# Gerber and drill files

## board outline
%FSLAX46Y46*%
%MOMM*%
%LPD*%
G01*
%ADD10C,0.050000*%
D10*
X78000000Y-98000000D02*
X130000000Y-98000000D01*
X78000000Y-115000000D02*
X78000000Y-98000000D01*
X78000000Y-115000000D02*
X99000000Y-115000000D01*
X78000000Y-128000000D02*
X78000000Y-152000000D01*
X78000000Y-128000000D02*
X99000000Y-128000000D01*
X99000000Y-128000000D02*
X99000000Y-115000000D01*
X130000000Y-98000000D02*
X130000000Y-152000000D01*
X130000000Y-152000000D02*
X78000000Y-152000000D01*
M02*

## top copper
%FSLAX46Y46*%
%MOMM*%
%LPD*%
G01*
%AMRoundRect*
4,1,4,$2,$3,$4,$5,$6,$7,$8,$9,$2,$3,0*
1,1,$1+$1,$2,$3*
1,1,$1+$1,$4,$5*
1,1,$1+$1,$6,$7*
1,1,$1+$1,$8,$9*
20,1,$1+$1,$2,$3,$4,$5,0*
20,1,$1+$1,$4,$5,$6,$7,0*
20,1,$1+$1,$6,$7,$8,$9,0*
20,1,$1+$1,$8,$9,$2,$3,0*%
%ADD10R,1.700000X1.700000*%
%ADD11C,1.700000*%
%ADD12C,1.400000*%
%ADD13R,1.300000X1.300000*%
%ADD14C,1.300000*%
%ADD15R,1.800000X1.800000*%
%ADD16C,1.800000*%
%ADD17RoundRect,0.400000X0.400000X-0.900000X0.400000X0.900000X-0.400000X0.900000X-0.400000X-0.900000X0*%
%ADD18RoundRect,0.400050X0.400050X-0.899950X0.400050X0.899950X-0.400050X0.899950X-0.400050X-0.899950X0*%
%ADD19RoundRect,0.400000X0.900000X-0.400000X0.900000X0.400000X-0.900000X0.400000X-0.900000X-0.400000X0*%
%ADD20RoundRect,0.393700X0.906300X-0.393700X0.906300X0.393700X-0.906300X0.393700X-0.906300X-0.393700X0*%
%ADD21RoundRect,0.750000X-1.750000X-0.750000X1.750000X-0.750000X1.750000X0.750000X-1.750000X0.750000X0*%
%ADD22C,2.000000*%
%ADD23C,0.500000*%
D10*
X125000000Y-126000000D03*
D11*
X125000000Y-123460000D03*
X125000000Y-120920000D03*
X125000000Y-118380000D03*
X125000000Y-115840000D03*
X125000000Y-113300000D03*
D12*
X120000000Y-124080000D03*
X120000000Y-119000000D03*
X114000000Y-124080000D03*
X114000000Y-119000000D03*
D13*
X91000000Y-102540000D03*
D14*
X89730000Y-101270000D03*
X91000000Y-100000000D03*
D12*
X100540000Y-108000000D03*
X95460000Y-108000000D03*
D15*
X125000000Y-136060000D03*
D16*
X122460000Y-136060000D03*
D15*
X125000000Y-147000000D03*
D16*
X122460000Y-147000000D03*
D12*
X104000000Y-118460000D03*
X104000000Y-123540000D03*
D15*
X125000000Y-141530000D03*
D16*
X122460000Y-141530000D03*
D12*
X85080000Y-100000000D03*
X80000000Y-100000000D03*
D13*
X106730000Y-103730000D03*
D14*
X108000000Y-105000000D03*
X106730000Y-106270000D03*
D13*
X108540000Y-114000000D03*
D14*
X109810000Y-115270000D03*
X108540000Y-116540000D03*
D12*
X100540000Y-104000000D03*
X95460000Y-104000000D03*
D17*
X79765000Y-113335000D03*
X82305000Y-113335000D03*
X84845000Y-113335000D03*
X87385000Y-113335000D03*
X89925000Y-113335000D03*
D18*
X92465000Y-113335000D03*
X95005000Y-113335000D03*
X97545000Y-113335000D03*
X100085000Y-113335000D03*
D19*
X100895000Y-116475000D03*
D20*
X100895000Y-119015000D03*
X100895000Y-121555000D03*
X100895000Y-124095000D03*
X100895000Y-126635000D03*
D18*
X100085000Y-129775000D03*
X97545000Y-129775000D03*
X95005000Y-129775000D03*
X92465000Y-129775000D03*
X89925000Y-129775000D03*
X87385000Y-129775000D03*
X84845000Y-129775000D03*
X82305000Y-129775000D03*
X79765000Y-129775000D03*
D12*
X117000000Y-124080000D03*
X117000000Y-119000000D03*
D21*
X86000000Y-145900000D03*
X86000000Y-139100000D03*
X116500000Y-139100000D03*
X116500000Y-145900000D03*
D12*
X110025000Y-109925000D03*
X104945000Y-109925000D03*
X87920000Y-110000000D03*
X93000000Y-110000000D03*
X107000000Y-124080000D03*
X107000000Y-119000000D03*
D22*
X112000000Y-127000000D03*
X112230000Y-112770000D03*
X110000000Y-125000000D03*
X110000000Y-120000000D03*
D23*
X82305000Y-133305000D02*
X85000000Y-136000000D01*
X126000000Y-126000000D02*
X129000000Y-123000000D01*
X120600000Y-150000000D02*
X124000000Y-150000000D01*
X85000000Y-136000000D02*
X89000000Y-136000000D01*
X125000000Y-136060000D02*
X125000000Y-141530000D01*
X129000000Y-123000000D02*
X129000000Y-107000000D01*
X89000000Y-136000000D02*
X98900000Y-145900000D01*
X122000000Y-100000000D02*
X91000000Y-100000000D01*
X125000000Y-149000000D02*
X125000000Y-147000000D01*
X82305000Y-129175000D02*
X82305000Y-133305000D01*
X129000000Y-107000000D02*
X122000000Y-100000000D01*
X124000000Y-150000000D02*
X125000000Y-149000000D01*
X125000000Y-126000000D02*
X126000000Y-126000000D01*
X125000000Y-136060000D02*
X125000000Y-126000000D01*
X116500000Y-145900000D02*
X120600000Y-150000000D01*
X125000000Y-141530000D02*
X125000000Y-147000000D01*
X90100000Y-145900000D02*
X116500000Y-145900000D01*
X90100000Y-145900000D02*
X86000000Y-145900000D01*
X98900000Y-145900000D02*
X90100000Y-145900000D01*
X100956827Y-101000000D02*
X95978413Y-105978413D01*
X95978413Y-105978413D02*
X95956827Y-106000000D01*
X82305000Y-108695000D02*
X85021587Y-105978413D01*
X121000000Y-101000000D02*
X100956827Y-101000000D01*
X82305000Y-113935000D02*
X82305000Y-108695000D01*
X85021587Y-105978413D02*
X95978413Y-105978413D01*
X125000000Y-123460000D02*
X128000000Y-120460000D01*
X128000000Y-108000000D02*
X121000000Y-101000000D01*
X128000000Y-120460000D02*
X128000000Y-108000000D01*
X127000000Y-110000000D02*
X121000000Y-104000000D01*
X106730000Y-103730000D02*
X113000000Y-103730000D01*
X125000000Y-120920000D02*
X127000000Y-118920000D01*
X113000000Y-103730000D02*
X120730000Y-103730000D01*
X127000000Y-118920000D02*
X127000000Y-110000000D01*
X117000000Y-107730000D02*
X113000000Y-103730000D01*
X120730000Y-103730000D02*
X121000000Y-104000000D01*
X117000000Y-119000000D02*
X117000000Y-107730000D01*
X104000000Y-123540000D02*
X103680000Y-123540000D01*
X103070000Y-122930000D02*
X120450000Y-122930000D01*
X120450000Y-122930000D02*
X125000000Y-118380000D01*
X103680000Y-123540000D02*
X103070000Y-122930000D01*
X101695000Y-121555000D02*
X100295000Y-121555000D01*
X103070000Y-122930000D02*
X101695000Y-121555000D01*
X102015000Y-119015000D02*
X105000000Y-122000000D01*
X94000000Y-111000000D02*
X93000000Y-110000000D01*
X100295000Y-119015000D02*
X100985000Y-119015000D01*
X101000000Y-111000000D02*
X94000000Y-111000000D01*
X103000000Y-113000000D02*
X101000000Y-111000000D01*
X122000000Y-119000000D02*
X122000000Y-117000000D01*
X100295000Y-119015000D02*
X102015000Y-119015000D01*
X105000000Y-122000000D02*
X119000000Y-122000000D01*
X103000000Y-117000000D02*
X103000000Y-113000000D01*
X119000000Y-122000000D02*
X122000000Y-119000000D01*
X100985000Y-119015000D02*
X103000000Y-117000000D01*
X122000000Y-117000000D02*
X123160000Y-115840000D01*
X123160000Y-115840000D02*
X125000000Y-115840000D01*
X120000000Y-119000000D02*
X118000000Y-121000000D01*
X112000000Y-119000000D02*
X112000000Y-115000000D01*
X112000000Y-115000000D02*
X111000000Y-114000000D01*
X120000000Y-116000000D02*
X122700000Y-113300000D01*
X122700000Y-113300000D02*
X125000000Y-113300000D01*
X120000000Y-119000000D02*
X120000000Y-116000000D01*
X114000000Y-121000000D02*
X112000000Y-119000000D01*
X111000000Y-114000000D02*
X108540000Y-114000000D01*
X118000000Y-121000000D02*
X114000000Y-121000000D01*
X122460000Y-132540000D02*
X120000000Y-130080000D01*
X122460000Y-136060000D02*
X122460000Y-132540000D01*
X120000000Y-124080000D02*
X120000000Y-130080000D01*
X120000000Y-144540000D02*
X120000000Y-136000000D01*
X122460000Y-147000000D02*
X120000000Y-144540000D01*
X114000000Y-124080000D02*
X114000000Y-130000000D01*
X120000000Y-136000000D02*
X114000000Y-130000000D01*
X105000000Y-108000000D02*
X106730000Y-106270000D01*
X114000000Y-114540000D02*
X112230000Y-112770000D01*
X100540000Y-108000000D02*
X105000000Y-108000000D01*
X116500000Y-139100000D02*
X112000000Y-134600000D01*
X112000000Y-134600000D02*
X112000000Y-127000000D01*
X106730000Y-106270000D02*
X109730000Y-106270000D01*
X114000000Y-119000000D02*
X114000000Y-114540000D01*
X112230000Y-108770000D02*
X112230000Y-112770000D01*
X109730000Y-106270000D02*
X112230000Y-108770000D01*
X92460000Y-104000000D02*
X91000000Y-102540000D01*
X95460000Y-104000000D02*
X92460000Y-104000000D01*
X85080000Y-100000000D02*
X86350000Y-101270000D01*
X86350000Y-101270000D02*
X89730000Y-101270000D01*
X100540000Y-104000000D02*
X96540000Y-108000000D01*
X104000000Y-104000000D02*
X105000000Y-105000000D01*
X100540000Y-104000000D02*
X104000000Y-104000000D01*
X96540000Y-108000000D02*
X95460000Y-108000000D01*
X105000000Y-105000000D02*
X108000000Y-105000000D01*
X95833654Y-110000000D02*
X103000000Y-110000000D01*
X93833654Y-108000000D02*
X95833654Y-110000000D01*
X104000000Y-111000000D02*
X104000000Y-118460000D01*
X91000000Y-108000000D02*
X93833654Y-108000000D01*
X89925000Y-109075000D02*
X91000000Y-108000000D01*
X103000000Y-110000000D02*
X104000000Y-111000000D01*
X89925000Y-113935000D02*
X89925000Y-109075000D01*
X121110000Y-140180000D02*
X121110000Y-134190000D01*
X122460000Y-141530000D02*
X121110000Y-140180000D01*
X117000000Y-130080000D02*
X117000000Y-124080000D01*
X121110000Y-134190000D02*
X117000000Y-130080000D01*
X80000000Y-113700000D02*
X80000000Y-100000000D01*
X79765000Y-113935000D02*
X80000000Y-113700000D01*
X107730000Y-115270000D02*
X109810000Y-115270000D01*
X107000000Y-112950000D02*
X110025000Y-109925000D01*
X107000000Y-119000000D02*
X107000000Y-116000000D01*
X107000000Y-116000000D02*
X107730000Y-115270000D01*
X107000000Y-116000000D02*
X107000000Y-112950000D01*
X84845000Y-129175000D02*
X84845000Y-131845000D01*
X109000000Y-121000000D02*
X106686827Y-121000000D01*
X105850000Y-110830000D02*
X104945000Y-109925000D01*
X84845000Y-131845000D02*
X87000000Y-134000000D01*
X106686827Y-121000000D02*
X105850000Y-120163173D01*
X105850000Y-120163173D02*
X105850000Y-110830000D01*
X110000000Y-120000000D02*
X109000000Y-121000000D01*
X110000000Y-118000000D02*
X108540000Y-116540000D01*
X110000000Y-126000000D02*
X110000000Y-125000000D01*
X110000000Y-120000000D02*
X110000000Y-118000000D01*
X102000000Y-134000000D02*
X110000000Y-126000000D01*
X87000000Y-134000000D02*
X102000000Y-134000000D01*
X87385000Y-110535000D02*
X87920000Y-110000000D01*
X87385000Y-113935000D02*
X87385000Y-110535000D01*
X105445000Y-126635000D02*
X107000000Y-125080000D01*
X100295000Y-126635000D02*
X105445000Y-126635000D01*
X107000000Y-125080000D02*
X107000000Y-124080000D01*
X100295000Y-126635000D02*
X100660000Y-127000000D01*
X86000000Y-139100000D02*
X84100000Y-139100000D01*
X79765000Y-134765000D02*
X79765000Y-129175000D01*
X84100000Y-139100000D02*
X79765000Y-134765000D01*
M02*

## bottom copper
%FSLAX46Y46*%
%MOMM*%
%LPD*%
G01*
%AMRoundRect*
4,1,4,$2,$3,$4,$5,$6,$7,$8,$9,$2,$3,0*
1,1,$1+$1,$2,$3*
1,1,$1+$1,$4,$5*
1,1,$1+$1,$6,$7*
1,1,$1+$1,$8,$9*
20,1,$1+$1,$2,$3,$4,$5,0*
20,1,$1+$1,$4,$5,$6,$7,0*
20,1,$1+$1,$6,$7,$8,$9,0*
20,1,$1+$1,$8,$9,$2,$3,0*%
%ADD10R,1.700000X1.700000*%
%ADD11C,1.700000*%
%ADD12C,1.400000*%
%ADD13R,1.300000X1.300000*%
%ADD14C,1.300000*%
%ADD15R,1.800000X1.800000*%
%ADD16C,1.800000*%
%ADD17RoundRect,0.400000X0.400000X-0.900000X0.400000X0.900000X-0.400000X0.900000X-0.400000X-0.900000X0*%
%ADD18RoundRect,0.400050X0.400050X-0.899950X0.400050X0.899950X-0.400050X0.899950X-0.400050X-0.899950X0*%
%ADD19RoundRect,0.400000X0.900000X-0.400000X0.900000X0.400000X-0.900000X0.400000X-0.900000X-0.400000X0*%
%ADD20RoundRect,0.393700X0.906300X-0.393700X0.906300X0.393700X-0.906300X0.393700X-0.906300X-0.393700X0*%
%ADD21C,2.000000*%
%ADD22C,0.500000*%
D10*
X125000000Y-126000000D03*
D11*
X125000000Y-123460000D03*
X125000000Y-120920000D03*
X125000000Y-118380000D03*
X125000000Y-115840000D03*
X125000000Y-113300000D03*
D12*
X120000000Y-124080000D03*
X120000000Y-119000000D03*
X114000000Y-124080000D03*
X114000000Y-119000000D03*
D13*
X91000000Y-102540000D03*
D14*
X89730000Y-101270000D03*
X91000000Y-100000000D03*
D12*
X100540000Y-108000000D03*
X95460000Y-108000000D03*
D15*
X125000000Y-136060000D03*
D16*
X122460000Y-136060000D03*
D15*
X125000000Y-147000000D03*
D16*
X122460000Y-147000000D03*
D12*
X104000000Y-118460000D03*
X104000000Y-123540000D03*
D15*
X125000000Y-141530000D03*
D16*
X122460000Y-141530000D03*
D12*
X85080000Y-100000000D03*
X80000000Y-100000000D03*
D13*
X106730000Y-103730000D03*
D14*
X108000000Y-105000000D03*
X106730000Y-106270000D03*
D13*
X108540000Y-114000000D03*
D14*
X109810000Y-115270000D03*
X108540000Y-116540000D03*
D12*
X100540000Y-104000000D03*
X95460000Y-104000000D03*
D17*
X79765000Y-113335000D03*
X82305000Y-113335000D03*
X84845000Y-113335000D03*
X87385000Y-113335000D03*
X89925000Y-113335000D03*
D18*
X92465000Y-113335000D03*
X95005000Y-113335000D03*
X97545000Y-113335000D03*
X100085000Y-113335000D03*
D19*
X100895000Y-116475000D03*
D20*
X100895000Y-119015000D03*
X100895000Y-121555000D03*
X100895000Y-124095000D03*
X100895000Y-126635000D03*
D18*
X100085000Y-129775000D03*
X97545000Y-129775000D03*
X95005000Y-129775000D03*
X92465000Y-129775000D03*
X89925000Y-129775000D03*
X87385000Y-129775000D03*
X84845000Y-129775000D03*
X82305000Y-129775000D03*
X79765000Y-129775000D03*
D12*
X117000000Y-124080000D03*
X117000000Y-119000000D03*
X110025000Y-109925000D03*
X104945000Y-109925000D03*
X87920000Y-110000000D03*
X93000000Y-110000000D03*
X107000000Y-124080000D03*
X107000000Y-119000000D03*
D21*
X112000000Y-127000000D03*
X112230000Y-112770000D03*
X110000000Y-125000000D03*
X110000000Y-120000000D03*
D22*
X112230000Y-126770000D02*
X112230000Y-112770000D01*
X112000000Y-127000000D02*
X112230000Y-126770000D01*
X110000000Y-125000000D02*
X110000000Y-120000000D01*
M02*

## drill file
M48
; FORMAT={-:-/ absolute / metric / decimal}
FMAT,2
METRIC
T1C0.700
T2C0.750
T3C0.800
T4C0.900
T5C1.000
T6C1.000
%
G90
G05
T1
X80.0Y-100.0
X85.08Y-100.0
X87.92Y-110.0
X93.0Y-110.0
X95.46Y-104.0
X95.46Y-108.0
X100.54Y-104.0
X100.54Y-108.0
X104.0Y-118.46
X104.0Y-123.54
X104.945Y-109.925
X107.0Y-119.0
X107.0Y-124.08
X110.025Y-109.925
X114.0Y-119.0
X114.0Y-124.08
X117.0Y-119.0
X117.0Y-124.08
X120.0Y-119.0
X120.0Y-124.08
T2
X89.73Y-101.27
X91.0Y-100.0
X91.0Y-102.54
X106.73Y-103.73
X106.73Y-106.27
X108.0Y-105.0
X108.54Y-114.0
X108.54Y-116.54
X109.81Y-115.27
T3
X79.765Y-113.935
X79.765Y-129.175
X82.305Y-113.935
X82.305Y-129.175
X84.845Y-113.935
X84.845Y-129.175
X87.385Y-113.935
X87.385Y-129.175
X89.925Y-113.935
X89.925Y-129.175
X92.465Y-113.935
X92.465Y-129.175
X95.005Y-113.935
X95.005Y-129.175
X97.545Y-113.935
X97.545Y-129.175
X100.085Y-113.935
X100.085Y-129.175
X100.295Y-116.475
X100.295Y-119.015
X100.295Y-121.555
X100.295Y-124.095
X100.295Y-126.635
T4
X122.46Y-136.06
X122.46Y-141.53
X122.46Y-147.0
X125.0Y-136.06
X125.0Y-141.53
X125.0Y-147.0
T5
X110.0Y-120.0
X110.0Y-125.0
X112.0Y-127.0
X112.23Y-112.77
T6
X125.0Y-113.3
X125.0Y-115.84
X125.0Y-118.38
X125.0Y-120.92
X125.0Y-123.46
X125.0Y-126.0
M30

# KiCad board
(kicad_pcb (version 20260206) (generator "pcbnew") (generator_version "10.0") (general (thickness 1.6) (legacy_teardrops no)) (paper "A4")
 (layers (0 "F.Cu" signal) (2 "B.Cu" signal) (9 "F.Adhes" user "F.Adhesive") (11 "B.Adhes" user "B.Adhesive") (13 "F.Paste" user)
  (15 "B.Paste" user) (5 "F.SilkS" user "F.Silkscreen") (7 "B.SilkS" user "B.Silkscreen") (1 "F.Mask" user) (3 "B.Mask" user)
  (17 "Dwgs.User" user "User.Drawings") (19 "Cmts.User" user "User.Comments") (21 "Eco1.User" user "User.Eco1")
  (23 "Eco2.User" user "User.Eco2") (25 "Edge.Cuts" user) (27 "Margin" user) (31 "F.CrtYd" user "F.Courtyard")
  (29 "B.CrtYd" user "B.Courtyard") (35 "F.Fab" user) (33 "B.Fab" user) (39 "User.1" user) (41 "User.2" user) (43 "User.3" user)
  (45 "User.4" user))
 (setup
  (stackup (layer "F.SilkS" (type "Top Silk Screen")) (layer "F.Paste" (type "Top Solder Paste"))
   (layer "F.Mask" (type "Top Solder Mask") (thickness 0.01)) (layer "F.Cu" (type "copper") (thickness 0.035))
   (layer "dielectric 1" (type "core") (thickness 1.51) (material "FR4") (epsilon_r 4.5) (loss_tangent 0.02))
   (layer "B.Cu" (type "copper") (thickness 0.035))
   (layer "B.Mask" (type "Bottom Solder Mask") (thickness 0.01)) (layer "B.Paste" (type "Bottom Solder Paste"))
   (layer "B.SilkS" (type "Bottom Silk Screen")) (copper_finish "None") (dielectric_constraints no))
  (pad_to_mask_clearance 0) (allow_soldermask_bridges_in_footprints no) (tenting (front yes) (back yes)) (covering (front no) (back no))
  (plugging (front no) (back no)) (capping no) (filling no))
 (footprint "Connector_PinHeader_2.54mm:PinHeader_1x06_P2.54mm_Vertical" (layer "F.Cu") (at 125 126 180)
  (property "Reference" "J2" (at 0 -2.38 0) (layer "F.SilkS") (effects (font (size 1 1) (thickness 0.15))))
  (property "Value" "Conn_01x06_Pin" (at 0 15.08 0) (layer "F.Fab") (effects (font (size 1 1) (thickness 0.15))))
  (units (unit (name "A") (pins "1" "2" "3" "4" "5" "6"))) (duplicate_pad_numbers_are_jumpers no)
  (pad "1" thru_hole rect (at 0 0 180) (size 1.7 1.7) (drill 1) (layers "*.Cu" "*.Mask") (remove_unused_layers no) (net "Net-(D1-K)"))
  (pad "2" thru_hole circle (at 0 2.54 180) (size 1.7 1.7) (drill 1) (layers "*.Cu" "*.Mask") (remove_unused_layers no)
   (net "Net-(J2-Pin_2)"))
  (pad "3" thru_hole circle (at 0 5.08 180) (size 1.7 1.7) (drill 1) (layers "*.Cu" "*.Mask") (remove_unused_layers no)
   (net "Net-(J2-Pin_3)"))
  (pad "4" thru_hole circle (at 0 7.62 180) (size 1.7 1.7) (drill 1) (layers "*.Cu" "*.Mask") (remove_unused_layers no)
   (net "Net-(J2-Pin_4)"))
  (pad "5" thru_hole circle (at 0 10.16 180) (size 1.7 1.7) (drill 1) (layers "*.Cu" "*.Mask") (remove_unused_layers no)
   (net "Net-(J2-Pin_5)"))
  (pad "6" thru_hole circle (at 0 12.7 180) (size 1.7 1.7) (drill 1) (layers "*.Cu" "*.Mask") (remove_unused_layers no)
   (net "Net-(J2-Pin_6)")))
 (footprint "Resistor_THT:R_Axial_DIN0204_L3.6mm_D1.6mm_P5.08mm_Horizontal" (layer "F.Cu") (at 120 124.08 90)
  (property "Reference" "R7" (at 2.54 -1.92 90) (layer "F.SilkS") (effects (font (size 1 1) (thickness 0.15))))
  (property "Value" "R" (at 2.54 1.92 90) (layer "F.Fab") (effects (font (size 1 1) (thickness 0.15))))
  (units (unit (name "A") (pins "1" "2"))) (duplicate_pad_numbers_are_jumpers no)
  (pad "1" thru_hole circle (at 0 0 90) (size 1.4 1.4) (drill 0.7) (layers "*.Cu" "*.Mask") (remove_unused_layers no) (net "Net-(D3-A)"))
  (pad "2" thru_hole circle (at 5.08 0 90) (size 1.4 1.4) (drill 0.7) (layers "*.Cu" "*.Mask") (remove_unused_layers no)
   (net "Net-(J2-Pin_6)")))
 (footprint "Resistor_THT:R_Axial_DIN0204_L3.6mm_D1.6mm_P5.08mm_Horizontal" (layer "F.Cu") (at 114 124.08 90)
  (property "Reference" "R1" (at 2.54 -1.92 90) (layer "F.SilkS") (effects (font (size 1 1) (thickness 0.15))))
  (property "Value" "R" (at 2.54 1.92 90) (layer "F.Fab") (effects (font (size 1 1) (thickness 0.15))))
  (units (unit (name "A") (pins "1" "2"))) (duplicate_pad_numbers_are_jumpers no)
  (pad "1" thru_hole circle (at 0 0 90) (size 1.4 1.4) (drill 0.7) (layers "*.Cu" "*.Mask") (remove_unused_layers no) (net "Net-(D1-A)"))
  (pad "2" thru_hole circle (at 5.08 0 90) (size 1.4 1.4) (drill 0.7) (layers "*.Cu" "*.Mask") (remove_unused_layers no)
   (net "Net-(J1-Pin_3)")))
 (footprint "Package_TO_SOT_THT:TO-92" (layer "F.Cu") (at 91 102.54 90)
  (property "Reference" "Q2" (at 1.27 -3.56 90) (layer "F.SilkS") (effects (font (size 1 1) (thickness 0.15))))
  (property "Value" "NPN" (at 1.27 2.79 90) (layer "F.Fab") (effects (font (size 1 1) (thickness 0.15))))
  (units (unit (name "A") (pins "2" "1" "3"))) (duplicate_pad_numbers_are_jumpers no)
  (pad "1" thru_hole rect (at 0 0 90) (size 1.3 1.3) (drill 0.75) (layers "*.Cu" "*.Mask") (remove_unused_layers no) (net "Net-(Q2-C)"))
  (pad "2" thru_hole circle (at 1.27 -1.27 90) (size 1.3 1.3) (drill 0.75) (layers "*.Cu" "*.Mask") (remove_unused_layers no)
   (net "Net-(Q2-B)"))
  (pad "3" thru_hole circle (at 2.54 0 90) (size 1.3 1.3) (drill 0.75) (layers "*.Cu" "*.Mask") (remove_unused_layers no) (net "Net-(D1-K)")))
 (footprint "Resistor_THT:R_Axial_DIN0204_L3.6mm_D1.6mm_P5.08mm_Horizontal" (layer "F.Cu") (at 100.54 108 180)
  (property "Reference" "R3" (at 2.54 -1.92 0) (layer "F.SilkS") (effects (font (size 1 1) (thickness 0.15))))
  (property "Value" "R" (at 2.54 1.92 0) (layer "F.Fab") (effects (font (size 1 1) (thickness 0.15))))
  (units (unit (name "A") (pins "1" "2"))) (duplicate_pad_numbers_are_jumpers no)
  (pad "1" thru_hole circle (at 0 0 180) (size 1.4 1.4) (drill 0.7) (layers "*.Cu" "*.Mask") (remove_unused_layers no)
   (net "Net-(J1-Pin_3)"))
  (pad "2" thru_hole circle (at 5.08 0 180) (size 1.4 1.4) (drill 0.7) (layers "*.Cu" "*.Mask") (remove_unused_layers no) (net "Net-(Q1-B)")))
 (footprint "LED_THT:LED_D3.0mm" (layer "F.Cu") (at 125 136.06 180)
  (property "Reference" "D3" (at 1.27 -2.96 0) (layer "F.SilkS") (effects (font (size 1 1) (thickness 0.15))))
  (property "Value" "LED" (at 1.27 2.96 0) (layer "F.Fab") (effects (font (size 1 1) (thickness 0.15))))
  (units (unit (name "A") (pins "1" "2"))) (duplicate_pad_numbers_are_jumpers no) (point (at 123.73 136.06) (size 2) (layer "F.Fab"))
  (pad "1" thru_hole rect (at 0 0 180) (size 1.8 1.8) (drill 0.9) (layers "*.Cu" "*.Mask") (remove_unused_layers no) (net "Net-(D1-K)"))
  (pad "2" thru_hole circle (at 2.54 0 180) (size 1.8 1.8) (drill 0.9) (layers "*.Cu" "*.Mask") (remove_unused_layers no) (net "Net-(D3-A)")))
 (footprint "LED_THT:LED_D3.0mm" (layer "F.Cu") (at 125 147 180)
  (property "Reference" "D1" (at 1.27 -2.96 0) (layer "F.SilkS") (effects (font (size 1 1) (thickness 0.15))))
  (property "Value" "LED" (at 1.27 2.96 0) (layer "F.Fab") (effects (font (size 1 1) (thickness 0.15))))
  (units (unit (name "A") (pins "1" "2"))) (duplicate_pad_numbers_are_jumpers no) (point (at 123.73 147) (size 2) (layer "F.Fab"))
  (pad "1" thru_hole rect (at 0 0 180) (size 1.8 1.8) (drill 0.9) (layers "*.Cu" "*.Mask") (remove_unused_layers no) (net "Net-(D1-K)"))
  (pad "2" thru_hole circle (at 2.54 0 180) (size 1.8 1.8) (drill 0.9) (layers "*.Cu" "*.Mask") (remove_unused_layers no) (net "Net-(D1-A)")))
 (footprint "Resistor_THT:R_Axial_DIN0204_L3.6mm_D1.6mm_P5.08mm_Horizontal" (layer "F.Cu") (at 104 118.46 -90)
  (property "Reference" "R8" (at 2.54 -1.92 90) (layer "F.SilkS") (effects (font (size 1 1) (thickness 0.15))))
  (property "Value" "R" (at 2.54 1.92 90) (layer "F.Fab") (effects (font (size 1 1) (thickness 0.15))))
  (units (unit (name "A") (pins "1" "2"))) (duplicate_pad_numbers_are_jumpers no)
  (pad "1" thru_hole circle (at 0 0 270) (size 1.4 1.4) (drill 0.7) (layers "*.Cu" "*.Mask") (remove_unused_layers no) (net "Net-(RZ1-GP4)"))
  (pad "2" thru_hole circle (at 5.08 0 270) (size 1.4 1.4) (drill 0.7) (layers "*.Cu" "*.Mask") (remove_unused_layers no)
   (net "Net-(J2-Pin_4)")))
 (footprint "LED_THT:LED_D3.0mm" (layer "F.Cu") (at 125 141.53 180)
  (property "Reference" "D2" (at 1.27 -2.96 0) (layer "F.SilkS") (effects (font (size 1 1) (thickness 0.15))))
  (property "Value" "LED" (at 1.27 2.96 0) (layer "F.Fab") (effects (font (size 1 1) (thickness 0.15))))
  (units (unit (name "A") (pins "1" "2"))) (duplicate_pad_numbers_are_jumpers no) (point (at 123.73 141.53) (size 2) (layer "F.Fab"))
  (pad "1" thru_hole rect (at 0 0 180) (size 1.8 1.8) (drill 0.9) (layers "*.Cu" "*.Mask") (remove_unused_layers no) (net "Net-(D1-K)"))
  (pad "2" thru_hole circle (at 2.54 0 180) (size 1.8 1.8) (drill 0.9) (layers "*.Cu" "*.Mask") (remove_unused_layers no) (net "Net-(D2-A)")))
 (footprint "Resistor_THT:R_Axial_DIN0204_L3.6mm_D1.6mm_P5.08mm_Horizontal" (layer "F.Cu") (at 85.08 100 180)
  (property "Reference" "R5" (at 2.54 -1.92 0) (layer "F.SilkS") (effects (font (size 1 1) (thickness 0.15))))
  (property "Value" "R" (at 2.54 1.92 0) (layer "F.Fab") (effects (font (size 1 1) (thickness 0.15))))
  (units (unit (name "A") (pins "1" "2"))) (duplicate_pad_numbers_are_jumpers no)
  (pad "1" thru_hole circle (at 0 0 180) (size 1.4 1.4) (drill 0.7) (layers "*.Cu" "*.Mask") (remove_unused_layers no) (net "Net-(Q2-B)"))
  (pad "2" thru_hole circle (at 5.08 0 180) (size 1.4 1.4) (drill 0.7) (layers "*.Cu" "*.Mask") (remove_unused_layers no)
   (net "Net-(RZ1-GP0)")))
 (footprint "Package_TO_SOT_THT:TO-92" (layer "F.Cu") (at 106.73 103.73 -90)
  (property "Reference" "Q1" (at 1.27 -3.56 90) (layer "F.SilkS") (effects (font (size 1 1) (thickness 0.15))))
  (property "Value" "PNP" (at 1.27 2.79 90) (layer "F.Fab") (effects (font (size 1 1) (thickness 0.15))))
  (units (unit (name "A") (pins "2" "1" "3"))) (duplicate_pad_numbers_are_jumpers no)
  (pad "1" thru_hole rect (at 0 0 270) (size 1.3 1.3) (drill 0.75) (layers "*.Cu" "*.Mask") (remove_unused_layers no) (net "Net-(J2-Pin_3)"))
  (pad "2" thru_hole circle (at 1.27 -1.27 270) (size 1.3 1.3) (drill 0.75) (layers "*.Cu" "*.Mask") (remove_unused_layers no)
   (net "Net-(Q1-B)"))
  (pad "3" thru_hole circle (at 2.54 0 270) (size 1.3 1.3) (drill 0.75) (layers "*.Cu" "*.Mask") (remove_unused_layers no)
   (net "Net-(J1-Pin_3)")))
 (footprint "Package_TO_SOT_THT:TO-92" (layer "F.Cu") (at 108.54 114 -90)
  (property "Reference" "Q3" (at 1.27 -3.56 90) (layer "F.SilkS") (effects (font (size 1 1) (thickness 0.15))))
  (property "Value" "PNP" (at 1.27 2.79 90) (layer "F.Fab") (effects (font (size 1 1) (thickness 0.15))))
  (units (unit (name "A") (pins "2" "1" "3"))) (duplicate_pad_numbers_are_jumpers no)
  (pad "1" thru_hole rect (at 0 0 270) (size 1.3 1.3) (drill 0.75) (layers "*.Cu" "*.Mask") (remove_unused_layers no) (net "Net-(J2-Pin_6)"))
  (pad "2" thru_hole circle (at 1.27 -1.27 270) (size 1.3 1.3) (drill 0.75) (layers "*.Cu" "*.Mask") (remove_unused_layers no)
   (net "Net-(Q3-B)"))
  (pad "3" thru_hole circle (at 2.54 0 270) (size 1.3 1.3) (drill 0.75) (layers "*.Cu" "*.Mask") (remove_unused_layers no)
   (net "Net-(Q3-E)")))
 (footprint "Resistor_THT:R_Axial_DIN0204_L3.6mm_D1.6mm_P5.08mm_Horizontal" (layer "F.Cu") (at 100.54 104 180)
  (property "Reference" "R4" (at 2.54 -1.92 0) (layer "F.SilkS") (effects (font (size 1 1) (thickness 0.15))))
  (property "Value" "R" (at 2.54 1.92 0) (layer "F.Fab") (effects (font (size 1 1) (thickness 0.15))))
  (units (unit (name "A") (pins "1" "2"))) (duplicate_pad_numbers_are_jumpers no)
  (pad "1" thru_hole circle (at 0 0 180) (size 1.4 1.4) (drill 0.7) (layers "*.Cu" "*.Mask") (remove_unused_layers no) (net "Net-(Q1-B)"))
  (pad "2" thru_hole circle (at 5.08 0 180) (size 1.4 1.4) (drill 0.7) (layers "*.Cu" "*.Mask") (remove_unused_layers no) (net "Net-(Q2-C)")))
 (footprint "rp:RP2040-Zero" (layer "F.Cu") (at 102.625 131.715 90)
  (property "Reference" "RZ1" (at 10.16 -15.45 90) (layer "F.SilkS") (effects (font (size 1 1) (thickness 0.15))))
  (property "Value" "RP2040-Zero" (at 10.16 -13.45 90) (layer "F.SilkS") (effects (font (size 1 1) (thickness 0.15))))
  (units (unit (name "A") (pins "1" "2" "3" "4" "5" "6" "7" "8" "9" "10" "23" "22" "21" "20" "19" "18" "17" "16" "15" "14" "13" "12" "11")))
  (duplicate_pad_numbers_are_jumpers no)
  (pad "1" thru_hole roundrect (at 17.78 -22.86 90) (size 2.6 1.6) (drill 0.8 (offset 0.6 0)) (layers "*.Cu" "*.Mask")
   (remove_unused_layers no) (roundrect_rratio 0.25) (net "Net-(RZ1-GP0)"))
  (pad "2" thru_hole roundrect (at 17.78 -20.32 90) (size 2.6 1.6) (drill 0.8 (offset 0.6 0)) (layers "*.Cu" "*.Mask")
   (remove_unused_layers no) (roundrect_rratio 0.25) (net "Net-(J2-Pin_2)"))
  (pad "3" thru_hole roundrect (at 17.78 -17.78 90) (size 2.6 1.6) (drill 0.8 (offset 0.6 0)) (layers "*.Cu" "*.Mask")
   (remove_unused_layers no) (roundrect_rratio 0.25) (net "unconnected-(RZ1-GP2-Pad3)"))
  (pad "4" thru_hole roundrect (at 17.78 -15.24 90) (size 2.6 1.6) (drill 0.8 (offset 0.6 0)) (layers "*.Cu" "*.Mask")
   (remove_unused_layers no) (roundrect_rratio 0.25) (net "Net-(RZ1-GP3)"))
  (pad "5" thru_hole roundrect (at 17.78 -12.7 90) (size 2.6 1.6) (drill 0.8 (offset 0.6 0)) (layers "*.Cu" "*.Mask")
   (remove_unused_layers no) (roundrect_rratio 0.25) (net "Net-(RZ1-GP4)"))
  (pad "6" thru_hole roundrect (at 17.78 -10.16 90) (size 2.6 1.6002) (drill 0.8 (offset 0.6 0)) (layers "*.Cu" "*.Mask")
   (remove_unused_layers no) (roundrect_rratio 0.25) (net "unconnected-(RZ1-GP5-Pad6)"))
  (pad "7" thru_hole roundrect (at 17.78 -7.62 90) (size 2.6 1.6002) (drill 0.8 (offset 0.6 0)) (layers "*.Cu" "*.Mask")
   (remove_unused_layers no) (roundrect_rratio 0.25) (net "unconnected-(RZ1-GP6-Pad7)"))
  (pad "8" thru_hole roundrect (at 17.78 -5.08 90) (size 2.6 1.6002) (drill 0.8 (offset 0.6 0)) (layers "*.Cu" "*.Mask")
   (remove_unused_layers no) (roundrect_rratio 0.25) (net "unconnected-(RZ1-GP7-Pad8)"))
  (pad "9" thru_hole roundrect (at 17.78 -2.54 90) (size 2.6 1.6002) (drill 0.8 (offset 0.6 0)) (layers "*.Cu" "*.Mask")
   (remove_unused_layers no) (roundrect_rratio 0.25) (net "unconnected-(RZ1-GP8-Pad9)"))
  (pad "10" thru_hole roundrect (at 15.24 -2.33 90) (size 1.6 2.6) (drill 0.8 (offset 0 0.6)) (layers "*.Cu" "*.Mask")
   (remove_unused_layers no) (roundrect_rratio 0.25) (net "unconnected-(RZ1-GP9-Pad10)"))
  (pad "11" thru_hole roundrect (at 12.7 -2.33 90) (size 1.5748 2.6) (drill 0.8 (offset 0 0.6)) (layers "*.Cu" "*.Mask")
   (remove_unused_layers no) (roundrect_rratio 0.25) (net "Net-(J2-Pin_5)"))
  (pad "12" thru_hole roundrect (at 10.16 -2.33 90) (size 1.5748 2.6) (drill 0.8 (offset 0 0.6)) (layers "*.Cu" "*.Mask")
   (remove_unused_layers no) (roundrect_rratio 0.25) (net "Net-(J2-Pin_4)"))
  (pad "13" thru_hole roundrect (at 7.62 -2.33 90) (size 1.5748 2.6) (drill 0.8 (offset 0 0.6)) (layers "*.Cu" "*.Mask")
   (remove_unused_layers no) (roundrect_rratio 0.25) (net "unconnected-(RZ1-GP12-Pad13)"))
  (pad "14" thru_hole roundrect (at 5.08 -2.33 90) (size 1.5748 2.6) (drill 0.8 (offset 0 0.6)) (layers "*.Cu" "*.Mask")
   (remove_unused_layers no) (roundrect_rratio 0.25) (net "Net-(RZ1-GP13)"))
  (pad "15" thru_hole roundrect (at 2.54 -2.54 90) (size 2.6 1.6002) (drill 0.8 (offset -0.6 0)) (layers "*.Cu" "*.Mask")
   (remove_unused_layers no) (roundrect_rratio 0.25) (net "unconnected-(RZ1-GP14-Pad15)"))
  (pad "16" thru_hole roundrect (at 2.54 -5.08 90) (size 2.6 1.6002) (drill 0.8 (offset -0.6 0)) (layers "*.Cu" "*.Mask")
   (remove_unused_layers no) (roundrect_rratio 0.25) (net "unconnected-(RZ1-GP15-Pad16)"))
  (pad "17" thru_hole roundrect (at 2.54 -7.62 90) (size 2.6 1.6002) (drill 0.8 (offset -0.6 0)) (layers "*.Cu" "*.Mask")
   (remove_unused_layers no) (roundrect_rratio 0.25) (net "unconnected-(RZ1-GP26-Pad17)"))
  (pad "18" thru_hole roundrect (at 2.54 -10.16 90) (size 2.6 1.6002) (drill 0.8 (offset -0.6 0)) (layers "*.Cu" "*.Mask")
   (remove_unused_layers no) (roundrect_rratio 0.25) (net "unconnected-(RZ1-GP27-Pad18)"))
  (pad "19" thru_hole roundrect (at 2.54 -12.7 90) (size 2.6 1.6002) (drill 0.8 (offset -0.6 0)) (layers "*.Cu" "*.Mask")
   (remove_unused_layers no) (roundrect_rratio 0.25) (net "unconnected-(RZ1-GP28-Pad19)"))
  (pad "20" thru_hole roundrect (at 2.54 -15.24 90) (size 2.6 1.6002) (drill 0.8 (offset -0.6 0)) (layers "*.Cu" "*.Mask")
   (remove_unused_layers no) (roundrect_rratio 0.25) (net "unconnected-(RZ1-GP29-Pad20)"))
  (pad "21" thru_hole roundrect (at 2.54 -17.78 90) (size 2.6 1.6002) (drill 0.8 (offset -0.6 0)) (layers "*.Cu" "*.Mask")
   (remove_unused_layers no) (roundrect_rratio 0.25) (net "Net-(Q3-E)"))
  (pad "22" thru_hole roundrect (at 2.54 -20.32 90) (size 2.6 1.6002) (drill 0.8 (offset -0.6 0)) (layers "*.Cu" "*.Mask")
   (remove_unused_layers no) (roundrect_rratio 0.25) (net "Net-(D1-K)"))
  (pad "23" thru_hole roundrect (at 2.54 -22.86 90) (size 2.6 1.6002) (drill 0.8 (offset -0.6 0)) (layers "*.Cu" "*.Mask")
   (remove_unused_layers no) (roundrect_rratio 0.25) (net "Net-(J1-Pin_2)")))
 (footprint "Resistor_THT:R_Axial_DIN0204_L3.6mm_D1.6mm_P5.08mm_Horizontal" (layer "F.Cu") (at 117 124.08 90)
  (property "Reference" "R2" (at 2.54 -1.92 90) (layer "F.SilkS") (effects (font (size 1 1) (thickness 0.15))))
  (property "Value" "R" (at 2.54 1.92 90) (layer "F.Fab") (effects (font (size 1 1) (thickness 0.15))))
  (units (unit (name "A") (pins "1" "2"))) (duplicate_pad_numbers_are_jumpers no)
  (pad "1" thru_hole circle (at 0 0 90) (size 1.4 1.4) (drill 0.7) (layers "*.Cu" "*.Mask") (remove_unused_layers no) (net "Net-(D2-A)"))
  (pad "2" thru_hole circle (at 5.08 0 90) (size 1.4 1.4) (drill 0.7) (layers "*.Cu" "*.Mask") (remove_unused_layers no)
   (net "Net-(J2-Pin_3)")))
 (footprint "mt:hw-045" (layer "F.Cu") (at 101 143)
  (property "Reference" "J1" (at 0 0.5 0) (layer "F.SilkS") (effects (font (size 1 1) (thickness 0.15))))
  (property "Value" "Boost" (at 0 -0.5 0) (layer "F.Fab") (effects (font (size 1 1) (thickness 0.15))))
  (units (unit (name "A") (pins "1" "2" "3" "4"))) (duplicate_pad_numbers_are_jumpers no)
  (pad "1" smd roundrect (at -15 2.9) (size 5 3) (layers "F.Cu" "F.Mask" "F.Paste") (roundrect_rratio 0.25) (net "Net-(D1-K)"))
  (pad "2" smd roundrect (at -15 -3.9) (size 5 3) (layers "F.Cu" "F.Mask" "F.Paste") (roundrect_rratio 0.25) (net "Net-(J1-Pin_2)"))
  (pad "3" smd roundrect (at 15.5 -3.9) (size 5 3) (layers "F.Cu" "F.Mask" "F.Paste") (roundrect_rratio 0.25) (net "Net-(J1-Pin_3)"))
  (pad "4" smd roundrect (at 15.5 2.9) (size 5 3) (layers "F.Cu" "F.Mask" "F.Paste") (roundrect_rratio 0.25) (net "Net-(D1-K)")))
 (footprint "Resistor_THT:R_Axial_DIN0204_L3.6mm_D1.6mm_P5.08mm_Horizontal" (layer "F.Cu") (at 110.025 109.925 180)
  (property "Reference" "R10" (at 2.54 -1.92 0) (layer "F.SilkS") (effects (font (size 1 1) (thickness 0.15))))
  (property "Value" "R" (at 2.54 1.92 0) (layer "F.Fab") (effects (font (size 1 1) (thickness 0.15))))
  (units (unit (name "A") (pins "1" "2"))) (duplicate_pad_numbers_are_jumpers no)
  (pad "1" thru_hole circle (at 0 0 180) (size 1.4 1.4) (drill 0.7) (layers "*.Cu" "*.Mask") (remove_unused_layers no) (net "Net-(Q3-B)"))
  (pad "2" thru_hole circle (at 5.08 0 180) (size 1.4 1.4) (drill 0.7) (layers "*.Cu" "*.Mask") (remove_unused_layers no) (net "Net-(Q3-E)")))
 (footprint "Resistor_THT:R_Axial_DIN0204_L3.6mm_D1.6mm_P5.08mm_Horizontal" (layer "F.Cu") (at 87.92 110)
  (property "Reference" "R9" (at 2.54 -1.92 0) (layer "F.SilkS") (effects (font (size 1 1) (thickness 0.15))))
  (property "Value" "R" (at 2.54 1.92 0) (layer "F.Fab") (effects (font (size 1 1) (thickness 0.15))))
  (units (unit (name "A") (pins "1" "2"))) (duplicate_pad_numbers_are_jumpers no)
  (pad "1" thru_hole circle (at 0 0) (size 1.4 1.4) (drill 0.7) (layers "*.Cu" "*.Mask") (remove_unused_layers no) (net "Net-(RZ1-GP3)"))
  (pad "2" thru_hole circle (at 5.08 0) (size 1.4 1.4) (drill 0.7) (layers "*.Cu" "*.Mask") (remove_unused_layers no) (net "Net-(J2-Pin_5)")))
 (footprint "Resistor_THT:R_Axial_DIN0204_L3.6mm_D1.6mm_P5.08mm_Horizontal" (layer "F.Cu") (at 107 124.08 90)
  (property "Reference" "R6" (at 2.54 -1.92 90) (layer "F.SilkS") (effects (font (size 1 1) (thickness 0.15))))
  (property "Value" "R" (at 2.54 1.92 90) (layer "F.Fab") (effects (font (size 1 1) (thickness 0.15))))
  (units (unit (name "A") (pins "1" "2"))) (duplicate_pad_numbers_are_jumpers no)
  (pad "1" thru_hole circle (at 0 0 90) (size 1.4 1.4) (drill 0.7) (layers "*.Cu" "*.Mask") (remove_unused_layers no) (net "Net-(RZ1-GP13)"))
  (pad "2" thru_hole circle (at 5.08 0 90) (size 1.4 1.4) (drill 0.7) (layers "*.Cu" "*.Mask") (remove_unused_layers no) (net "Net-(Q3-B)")))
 (gr_line (start 78 98) (end 130 98) (stroke (width 0.05) (type default)) (layer "Edge.Cuts"))
 (gr_line (start 78 115) (end 78 98) (stroke (width 0.05) (type default)) (layer "Edge.Cuts"))
 (gr_line (start 78 115) (end 99 115) (stroke (width 0.05) (type default)) (layer "Edge.Cuts"))
 (gr_line (start 78 128) (end 78 152) (stroke (width 0.05) (type default)) (layer "Edge.Cuts"))
 (gr_line (start 78 128) (end 99 128) (stroke (width 0.05) (type default)) (layer "Edge.Cuts"))
 (gr_line (start 99 128) (end 99 115) (stroke (width 0.05) (type default)) (layer "Edge.Cuts"))
 (gr_line (start 130 98) (end 130 152) (stroke (width 0.05) (type default)) (layer "Edge.Cuts"))
 (gr_line (start 130 152) (end 78 152) (stroke (width 0.05) (type default)) (layer "Edge.Cuts"))
 (segment (start 82.305 133.305) (end 85 136) (width 0.5) (layer "F.Cu") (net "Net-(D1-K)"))
 (segment (start 126 126) (end 129 123) (width 0.5) (layer "F.Cu") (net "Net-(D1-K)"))
 (segment (start 120.6 150) (end 124 150) (width 0.5) (layer "F.Cu") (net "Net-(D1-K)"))
 (segment (start 85 136) (end 89 136) (width 0.5) (layer "F.Cu") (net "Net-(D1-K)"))
 (segment (start 125 136.06) (end 125 141.53) (width 0.5) (layer "F.Cu") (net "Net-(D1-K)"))
 (segment (start 129 123) (end 129 107) (width 0.5) (layer "F.Cu") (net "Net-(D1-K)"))
 (segment (start 89 136) (end 98.9 145.9) (width 0.5) (layer "F.Cu") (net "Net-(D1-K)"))
 (segment (start 122 100) (end 91 100) (width 0.5) (layer "F.Cu") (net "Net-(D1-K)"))
 (segment (start 125 149) (end 125 147) (width 0.5) (layer "F.Cu") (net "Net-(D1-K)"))
 (segment (start 82.305 129.175) (end 82.305 133.305) (width 0.5) (layer "F.Cu") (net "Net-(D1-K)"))
 (segment (start 129 107) (end 122 100) (width 0.5) (layer "F.Cu") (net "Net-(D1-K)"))
 (segment (start 124 150) (end 125 149) (width 0.5) (layer "F.Cu") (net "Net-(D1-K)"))
 (segment (start 125 126) (end 126 126) (width 0.5) (layer "F.Cu") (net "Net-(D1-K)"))
 (segment (start 125 136.06) (end 125 126) (width 0.5) (layer "F.Cu") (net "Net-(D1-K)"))
 (segment (start 116.5 145.9) (end 120.6 150) (width 0.5) (layer "F.Cu") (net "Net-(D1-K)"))
 (segment (start 125 141.53) (end 125 147) (width 0.5) (layer "F.Cu") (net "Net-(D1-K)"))
 (segment (start 90.1 145.9) (end 116.5 145.9) (width 0.5) (layer "F.Cu") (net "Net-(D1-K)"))
 (segment (start 90.1 145.9) (end 86 145.9) (width 0.5) (layer "F.Cu") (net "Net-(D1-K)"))
 (segment (start 98.9 145.9) (end 90.1 145.9) (width 0.5) (layer "F.Cu") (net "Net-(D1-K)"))
 (segment (start 100.956827 101) (end 95.978413 105.978413) (width 0.5) (layer "F.Cu") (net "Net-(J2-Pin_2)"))
 (segment (start 95.978413 105.978413) (end 95.956827 106) (width 0.5) (layer "F.Cu") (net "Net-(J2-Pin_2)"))
 (segment (start 82.305 108.695) (end 85.021587 105.978413) (width 0.5) (layer "F.Cu") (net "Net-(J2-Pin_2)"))
 (segment (start 121 101) (end 100.956827 101) (width 0.5) (layer "F.Cu") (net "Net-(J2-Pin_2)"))
 (segment (start 82.305 113.935) (end 82.305 108.695) (width 0.5) (layer "F.Cu") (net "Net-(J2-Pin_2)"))
 (segment (start 85.021587 105.978413) (end 95.978413 105.978413) (width 0.5) (layer "F.Cu") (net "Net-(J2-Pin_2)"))
 (segment (start 125 123.46) (end 128 120.46) (width 0.5) (layer "F.Cu") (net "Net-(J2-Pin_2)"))
 (segment (start 128 108) (end 121 101) (width 0.5) (layer "F.Cu") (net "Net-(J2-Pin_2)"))
 (segment (start 128 120.46) (end 128 108) (width 0.5) (layer "F.Cu") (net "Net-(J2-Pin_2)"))
 (segment (start 127 110) (end 121 104) (width 0.5) (layer "F.Cu") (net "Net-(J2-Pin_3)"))
 (segment (start 106.73 103.73) (end 113 103.73) (width 0.5) (layer "F.Cu") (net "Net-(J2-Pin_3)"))
 (segment (start 125 120.92) (end 127 118.92) (width 0.5) (layer "F.Cu") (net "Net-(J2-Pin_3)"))
 (segment (start 113 103.73) (end 120.73 103.73) (width 0.5) (layer "F.Cu") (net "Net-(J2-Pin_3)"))
 (segment (start 127 118.92) (end 127 110) (width 0.5) (layer "F.Cu") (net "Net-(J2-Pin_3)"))
 (segment (start 117 107.73) (end 113 103.73) (width 0.5) (layer "F.Cu") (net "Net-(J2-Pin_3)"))
 (segment (start 120.73 103.73) (end 121 104) (width 0.5) (layer "F.Cu") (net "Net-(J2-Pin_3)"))
 (segment (start 117 119) (end 117 107.73) (width 0.5) (layer "F.Cu") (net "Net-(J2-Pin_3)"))
 (segment (start 104 123.54) (end 103.68 123.54) (width 0.5) (layer "F.Cu") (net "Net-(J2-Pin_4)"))
 (segment (start 103.07 122.93) (end 120.45 122.93) (width 0.5) (layer "F.Cu") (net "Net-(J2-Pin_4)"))
 (segment (start 120.45 122.93) (end 125 118.38) (width 0.5) (layer "F.Cu") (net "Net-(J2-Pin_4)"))
 (segment (start 103.68 123.54) (end 103.07 122.93) (width 0.5) (layer "F.Cu") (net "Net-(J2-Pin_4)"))
 (segment (start 101.695 121.555) (end 100.295 121.555) (width 0.5) (layer "F.Cu") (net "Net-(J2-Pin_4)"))
 (segment (start 103.07 122.93) (end 101.695 121.555) (width 0.5) (layer "F.Cu") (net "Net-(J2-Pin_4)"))
 (segment (start 102.015 119.015) (end 105 122) (width 0.5) (layer "F.Cu") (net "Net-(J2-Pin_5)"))
 (segment (start 94 111) (end 93 110) (width 0.5) (layer "F.Cu") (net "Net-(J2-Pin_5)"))
 (segment (start 100.295 119.015) (end 100.985 119.015) (width 0.5) (layer "F.Cu") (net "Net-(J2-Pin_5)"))
 (segment (start 101 111) (end 94 111) (width 0.5) (layer "F.Cu") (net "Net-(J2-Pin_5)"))
 (segment (start 103 113) (end 101 111) (width 0.5) (layer "F.Cu") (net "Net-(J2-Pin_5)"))
 (segment (start 122 119) (end 122 117) (width 0.5) (layer "F.Cu") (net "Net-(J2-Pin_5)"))
 (segment (start 100.295 119.015) (end 102.015 119.015) (width 0.5) (layer "F.Cu") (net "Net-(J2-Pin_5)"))
 (segment (start 105 122) (end 119 122) (width 0.5) (layer "F.Cu") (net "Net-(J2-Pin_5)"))
 (segment (start 103 117) (end 103 113) (width 0.5) (layer "F.Cu") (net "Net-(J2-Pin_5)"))
 (segment (start 119 122) (end 122 119) (width 0.5) (layer "F.Cu") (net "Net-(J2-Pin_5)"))
 (segment (start 100.985 119.015) (end 103 117) (width 0.5) (layer "F.Cu") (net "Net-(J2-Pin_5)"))
 (segment (start 122 117) (end 123.16 115.84) (width 0.5) (layer "F.Cu") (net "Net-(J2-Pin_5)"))
 (segment (start 123.16 115.84) (end 125 115.84) (width 0.5) (layer "F.Cu") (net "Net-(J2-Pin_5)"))
 (segment (start 120 119) (end 118 121) (width 0.5) (layer "F.Cu") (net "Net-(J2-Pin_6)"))
 (segment (start 112 119) (end 112 115) (width 0.5) (layer "F.Cu") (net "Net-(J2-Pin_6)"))
 (segment (start 112 115) (end 111 114) (width 0.5) (layer "F.Cu") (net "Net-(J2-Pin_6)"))
 (segment (start 120 116) (end 122.7 113.3) (width 0.5) (layer "F.Cu") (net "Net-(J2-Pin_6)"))
 (segment (start 122.7 113.3) (end 125 113.3) (width 0.5) (layer "F.Cu") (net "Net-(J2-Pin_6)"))
 (segment (start 120 119) (end 120 116) (width 0.5) (layer "F.Cu") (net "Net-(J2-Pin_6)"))
 (segment (start 114 121) (end 112 119) (width 0.5) (layer "F.Cu") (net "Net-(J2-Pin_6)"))
 (segment (start 111 114) (end 108.54 114) (width 0.5) (layer "F.Cu") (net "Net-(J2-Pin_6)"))
 (segment (start 118 121) (end 114 121) (width 0.5) (layer "F.Cu") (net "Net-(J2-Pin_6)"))
 (segment (start 122.46 132.54) (end 120 130.08) (width 0.5) (layer "F.Cu") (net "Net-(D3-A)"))
 (segment (start 122.46 136.06) (end 122.46 132.54) (width 0.5) (layer "F.Cu") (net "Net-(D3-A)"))
 (segment (start 120 124.08) (end 120 130.08) (width 0.5) (layer "F.Cu") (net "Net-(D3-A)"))
 (segment (start 120 144.54) (end 120 136) (width 0.5) (layer "F.Cu") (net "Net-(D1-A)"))
 (segment (start 122.46 147) (end 120 144.54) (width 0.5) (layer "F.Cu") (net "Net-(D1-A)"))
 (segment (start 114 124.08) (end 114 130) (width 0.5) (layer "F.Cu") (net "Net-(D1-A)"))
 (segment (start 120 136) (end 114 130) (width 0.5) (layer "F.Cu") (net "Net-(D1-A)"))
 (segment (start 105 108) (end 106.73 106.27) (width 0.5) (layer "F.Cu") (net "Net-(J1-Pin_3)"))
 (segment (start 114 114.54) (end 112.23 112.77) (width 0.5) (layer "F.Cu") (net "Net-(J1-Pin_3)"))
 (segment (start 100.54 108) (end 105 108) (width 0.5) (layer "F.Cu") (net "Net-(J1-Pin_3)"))
 (segment (start 116.5 139.1) (end 112 134.6) (width 0.5) (layer "F.Cu") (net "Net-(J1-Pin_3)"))
 (segment (start 112 134.6) (end 112 127) (width 0.5) (layer "F.Cu") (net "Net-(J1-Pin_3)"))
 (segment (start 106.73 106.27) (end 109.73 106.27) (width 0.5) (layer "F.Cu") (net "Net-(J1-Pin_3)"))
 (segment (start 114 119) (end 114 114.54) (width 0.5) (layer "F.Cu") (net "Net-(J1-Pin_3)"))
 (segment (start 112.23 108.77) (end 112.23 112.77) (width 0.5) (layer "F.Cu") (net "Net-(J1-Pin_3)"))
 (segment (start 109.73 106.27) (end 112.23 108.77) (width 0.5) (layer "F.Cu") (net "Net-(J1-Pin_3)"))
 (via (at 112 127) (size 2) (drill 1) (layers "F.Cu" "B.Cu") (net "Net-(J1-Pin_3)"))
 (via (at 112.23 112.77) (size 2) (drill 1) (layers "F.Cu" "B.Cu") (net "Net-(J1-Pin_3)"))
 (segment (start 112.23 126.77) (end 112.23 112.77) (width 0.5) (layer "B.Cu") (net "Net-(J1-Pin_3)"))
 (segment (start 112 127) (end 112.23 126.77) (width 0.5) (layer "B.Cu") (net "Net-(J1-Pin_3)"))
 (segment (start 92.46 104) (end 91 102.54) (width 0.5) (layer "F.Cu") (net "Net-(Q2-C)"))
 (segment (start 95.46 104) (end 92.46 104) (width 0.5) (layer "F.Cu") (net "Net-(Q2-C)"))
 (segment (start 85.08 100) (end 86.35 101.27) (width 0.5) (layer "F.Cu") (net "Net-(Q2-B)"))
 (segment (start 86.35 101.27) (end 89.73 101.27) (width 0.5) (layer "F.Cu") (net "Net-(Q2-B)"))
 (segment (start 100.54 104) (end 96.54 108) (width 0.5) (layer "F.Cu") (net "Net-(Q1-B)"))
 (segment (start 104 104) (end 105 105) (width 0.5) (layer "F.Cu") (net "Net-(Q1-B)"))
 (segment (start 100.54 104) (end 104 104) (width 0.5) (layer "F.Cu") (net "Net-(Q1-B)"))
 (segment (start 96.54 108) (end 95.46 108) (width 0.5) (layer "F.Cu") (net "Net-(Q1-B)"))
 (segment (start 105 105) (end 108 105) (width 0.5) (layer "F.Cu") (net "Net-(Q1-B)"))
 (segment (start 95.833654 110) (end 103 110) (width 0.5) (layer "F.Cu") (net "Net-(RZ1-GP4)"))
 (segment (start 93.833654 108) (end 95.833654 110) (width 0.5) (layer "F.Cu") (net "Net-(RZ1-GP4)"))
 (segment (start 104 111) (end 104 118.46) (width 0.5) (layer "F.Cu") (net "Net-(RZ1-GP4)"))
 (segment (start 91 108) (end 93.833654 108) (width 0.5) (layer "F.Cu") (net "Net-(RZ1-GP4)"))
 (segment (start 89.925 109.075) (end 91 108) (width 0.5) (layer "F.Cu") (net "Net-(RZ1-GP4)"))
 (segment (start 103 110) (end 104 111) (width 0.5) (layer "F.Cu") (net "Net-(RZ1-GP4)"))
 (segment (start 89.925 113.935) (end 89.925 109.075) (width 0.5) (layer "F.Cu") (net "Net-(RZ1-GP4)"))
 (segment (start 121.11 140.18) (end 121.11 134.19) (width 0.5) (layer "F.Cu") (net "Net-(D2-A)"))
 (segment (start 122.46 141.53) (end 121.11 140.18) (width 0.5) (layer "F.Cu") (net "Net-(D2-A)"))
 (segment (start 117 130.08) (end 117 124.08) (width 0.5) (layer "F.Cu") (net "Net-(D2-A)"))
 (segment (start 121.11 134.19) (end 117 130.08) (width 0.5) (layer "F.Cu") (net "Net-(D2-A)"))
 (segment (start 80 113.7) (end 80 100) (width 0.5) (layer "F.Cu") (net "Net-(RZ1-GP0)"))
 (segment (start 79.765 113.935) (end 80 113.7) (width 0.5) (layer "F.Cu") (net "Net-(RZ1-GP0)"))
 (segment (start 107.73 115.27) (end 109.81 115.27) (width 0.5) (layer "F.Cu") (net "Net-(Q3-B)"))
 (segment (start 107 112.95) (end 110.025 109.925) (width 0.5) (layer "F.Cu") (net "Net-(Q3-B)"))
 (segment (start 107 119) (end 107 116) (width 0.5) (layer "F.Cu") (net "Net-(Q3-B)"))
 (segment (start 107 116) (end 107.73 115.27) (width 0.5) (layer "F.Cu") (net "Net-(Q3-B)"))
 (segment (start 107 116) (end 107 112.95) (width 0.5) (layer "F.Cu") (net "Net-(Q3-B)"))
 (segment (start 84.845 129.175) (end 84.845 131.845) (width 0.5) (layer "F.Cu") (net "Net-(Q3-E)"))
 (segment (start 109 121) (end 106.686827 121) (width 0.5) (layer "F.Cu") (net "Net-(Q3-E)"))
 (segment (start 105.85 110.83) (end 104.945 109.925) (width 0.5) (layer "F.Cu") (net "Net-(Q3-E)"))
 (segment (start 84.845 131.845) (end 87 134) (width 0.5) (layer "F.Cu") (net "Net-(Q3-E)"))
 (segment (start 106.686827 121) (end 105.85 120.163173) (width 0.5) (layer "F.Cu") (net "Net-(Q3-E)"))
 (segment (start 105.85 120.163173) (end 105.85 110.83) (width 0.5) (layer "F.Cu") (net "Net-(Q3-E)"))
 (segment (start 110 120) (end 109 121) (width 0.5) (layer "F.Cu") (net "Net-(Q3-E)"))
 (segment (start 110 118) (end 108.54 116.54) (width 0.5) (layer "F.Cu") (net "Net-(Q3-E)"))
 (segment (start 110 126) (end 110 125) (width 0.5) (layer "F.Cu") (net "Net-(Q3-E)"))
 (segment (start 110 120) (end 110 118) (width 0.5) (layer "F.Cu") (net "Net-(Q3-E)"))
 (segment (start 102 134) (end 110 126) (width 0.5) (layer "F.Cu") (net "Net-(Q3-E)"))
 (segment (start 87 134) (end 102 134) (width 0.5) (layer "F.Cu") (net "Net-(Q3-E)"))
 (via (at 110 125) (size 2) (drill 1) (layers "F.Cu" "B.Cu") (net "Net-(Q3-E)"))
 (via (at 110 120) (size 2) (drill 1) (layers "F.Cu" "B.Cu") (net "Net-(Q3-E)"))
 (segment (start 110 125) (end 110 120) (width 0.5) (layer "B.Cu") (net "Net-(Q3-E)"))
 (segment (start 87.385 110.535) (end 87.92 110) (width 0.5) (layer "F.Cu") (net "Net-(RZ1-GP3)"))
 (segment (start 87.385 113.935) (end 87.385 110.535) (width 0.5) (layer "F.Cu") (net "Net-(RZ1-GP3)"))
 (segment (start 105.445 126.635) (end 107 125.08) (width 0.5) (layer "F.Cu") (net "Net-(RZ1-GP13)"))
 (segment (start 100.295 126.635) (end 105.445 126.635) (width 0.5) (layer "F.Cu") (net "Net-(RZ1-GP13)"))
 (segment (start 107 125.08) (end 107 124.08) (width 0.5) (layer "F.Cu") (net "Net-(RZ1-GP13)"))
 (segment (start 100.295 126.635) (end 100.66 127) (width 0.5) (layer "F.Cu") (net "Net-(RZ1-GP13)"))
 (segment (start 86 139.1) (end 84.1 139.1) (width 0.5) (layer "F.Cu") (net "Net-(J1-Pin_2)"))
 (segment (start 79.765 134.765) (end 79.765 129.175) (width 0.5) (layer "F.Cu") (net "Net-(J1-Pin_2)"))
 (segment (start 84.1 139.1) (end 79.765 134.765) (width 0.5) (layer "F.Cu") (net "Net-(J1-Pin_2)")))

